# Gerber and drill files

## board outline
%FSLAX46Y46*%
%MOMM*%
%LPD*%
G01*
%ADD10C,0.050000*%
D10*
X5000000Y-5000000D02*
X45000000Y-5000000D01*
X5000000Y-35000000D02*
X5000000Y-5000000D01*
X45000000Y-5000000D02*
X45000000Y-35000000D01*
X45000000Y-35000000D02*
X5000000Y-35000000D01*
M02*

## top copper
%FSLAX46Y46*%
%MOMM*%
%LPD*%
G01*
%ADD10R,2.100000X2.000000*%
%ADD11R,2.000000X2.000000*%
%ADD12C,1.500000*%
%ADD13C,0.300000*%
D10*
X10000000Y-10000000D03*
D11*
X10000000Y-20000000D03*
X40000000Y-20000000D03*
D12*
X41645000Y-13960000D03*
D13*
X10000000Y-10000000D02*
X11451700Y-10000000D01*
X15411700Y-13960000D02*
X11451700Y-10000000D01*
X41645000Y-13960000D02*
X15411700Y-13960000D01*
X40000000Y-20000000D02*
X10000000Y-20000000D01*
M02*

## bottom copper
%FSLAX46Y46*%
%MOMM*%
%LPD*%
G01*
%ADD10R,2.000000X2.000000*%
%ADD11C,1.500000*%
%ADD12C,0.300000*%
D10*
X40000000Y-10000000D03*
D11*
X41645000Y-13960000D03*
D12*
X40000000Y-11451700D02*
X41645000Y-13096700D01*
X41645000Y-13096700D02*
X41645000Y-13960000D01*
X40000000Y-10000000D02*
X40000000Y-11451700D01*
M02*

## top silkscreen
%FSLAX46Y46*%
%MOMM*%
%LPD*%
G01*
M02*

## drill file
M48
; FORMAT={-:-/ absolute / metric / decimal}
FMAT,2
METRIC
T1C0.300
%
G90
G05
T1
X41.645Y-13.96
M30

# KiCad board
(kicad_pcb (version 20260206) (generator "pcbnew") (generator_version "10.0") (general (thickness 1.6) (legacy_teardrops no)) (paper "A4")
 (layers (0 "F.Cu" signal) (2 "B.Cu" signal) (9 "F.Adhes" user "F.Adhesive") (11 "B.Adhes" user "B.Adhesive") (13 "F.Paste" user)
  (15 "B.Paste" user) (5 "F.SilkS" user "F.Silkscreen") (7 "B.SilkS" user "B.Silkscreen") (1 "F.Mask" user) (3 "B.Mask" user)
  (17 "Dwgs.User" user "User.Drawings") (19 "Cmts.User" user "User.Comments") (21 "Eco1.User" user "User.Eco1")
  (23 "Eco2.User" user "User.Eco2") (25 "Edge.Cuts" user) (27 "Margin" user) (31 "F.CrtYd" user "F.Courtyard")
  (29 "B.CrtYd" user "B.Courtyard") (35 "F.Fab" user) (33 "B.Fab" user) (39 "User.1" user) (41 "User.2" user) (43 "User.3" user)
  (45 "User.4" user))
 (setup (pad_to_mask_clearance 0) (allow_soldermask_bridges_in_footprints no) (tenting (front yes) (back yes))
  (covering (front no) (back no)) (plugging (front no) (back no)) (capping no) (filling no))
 (gr_line (start 5 5) (end 45 5) (stroke (width 0.05) (type default)) (layer "Edge.Cuts"))
 (gr_line (start 5 35) (end 5 5) (stroke (width 0.05) (type default)) (layer "Edge.Cuts"))
 (gr_line (start 45 5) (end 45 35) (stroke (width 0.05) (type default)) (layer "Edge.Cuts"))
 (gr_line (start 45 35) (end 5 35) (stroke (width 0.05) (type default)) (layer "Edge.Cuts"))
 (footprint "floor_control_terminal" (layer "F.Cu") (at 10 10)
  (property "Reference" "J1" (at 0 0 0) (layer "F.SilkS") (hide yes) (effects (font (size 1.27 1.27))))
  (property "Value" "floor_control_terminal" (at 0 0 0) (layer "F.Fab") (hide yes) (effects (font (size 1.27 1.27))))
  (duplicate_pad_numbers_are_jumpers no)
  (pad "1" smd rect (at 0 0) (size 2.1 2) (layers "F.Cu" "F.Paste" "F.Mask") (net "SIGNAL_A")))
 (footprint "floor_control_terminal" (layer "B.Cu") (at 40 10)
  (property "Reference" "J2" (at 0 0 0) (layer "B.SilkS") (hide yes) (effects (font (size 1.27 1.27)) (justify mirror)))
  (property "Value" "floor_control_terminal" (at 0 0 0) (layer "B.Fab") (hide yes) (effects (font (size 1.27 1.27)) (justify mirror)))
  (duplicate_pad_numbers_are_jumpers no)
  (pad "1" smd rect (at 0 0) (size 2 2) (layers "B.Cu" "B.Paste" "B.Mask") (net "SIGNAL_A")))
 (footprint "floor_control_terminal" (layer "F.Cu") (at 10 20)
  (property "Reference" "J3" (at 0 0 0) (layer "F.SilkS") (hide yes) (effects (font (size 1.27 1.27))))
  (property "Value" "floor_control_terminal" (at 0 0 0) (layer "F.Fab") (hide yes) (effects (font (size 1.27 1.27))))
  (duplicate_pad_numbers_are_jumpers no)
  (pad "1" smd rect (at 0 0) (size 2 2) (layers "F.Cu" "F.Paste" "F.Mask") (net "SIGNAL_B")))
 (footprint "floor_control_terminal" (layer "F.Cu") (at 40 20)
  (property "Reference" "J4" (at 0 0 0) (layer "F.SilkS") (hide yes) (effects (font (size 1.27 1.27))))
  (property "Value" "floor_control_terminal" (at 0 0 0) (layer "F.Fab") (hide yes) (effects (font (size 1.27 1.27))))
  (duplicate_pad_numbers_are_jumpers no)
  (pad "1" smd rect (at 0 0) (size 2 2) (layers "F.Cu" "F.Paste" "F.Mask") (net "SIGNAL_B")))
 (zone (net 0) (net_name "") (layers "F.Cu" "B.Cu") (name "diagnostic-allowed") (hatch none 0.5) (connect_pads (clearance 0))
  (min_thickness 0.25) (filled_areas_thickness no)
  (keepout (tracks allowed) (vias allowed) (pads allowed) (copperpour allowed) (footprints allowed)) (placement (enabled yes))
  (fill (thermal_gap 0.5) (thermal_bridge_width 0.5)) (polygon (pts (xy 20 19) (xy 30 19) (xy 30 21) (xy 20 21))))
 (segment (start 10 10) (end 11.4517 10) (width 0.3) (layer "F.Cu") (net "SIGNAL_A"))
 (segment (start 15.4117 13.96) (end 11.4517 10) (width 0.3) (layer "F.Cu") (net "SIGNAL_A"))
 (segment (start 41.645 13.96) (end 15.4117 13.96) (width 0.3) (layer "F.Cu") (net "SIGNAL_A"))
 (via (at 41.645 13.96) (size 1.5) (drill 0.3) (layers "F.Cu" "B.Cu") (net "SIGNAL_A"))
 (segment (start 40 11.4517) (end 41.645 13.0967) (width 0.3) (layer "B.Cu") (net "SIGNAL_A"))
 (segment (start 41.645 13.0967) (end 41.645 13.96) (width 0.3) (layer "B.Cu") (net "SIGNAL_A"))
 (segment (start 40 10) (end 40 11.4517) (width 0.3) (layer "B.Cu") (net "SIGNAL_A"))
 (segment (start 40 20) (end 10 20) (width 0.3) (layer "F.Cu") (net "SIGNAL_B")))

